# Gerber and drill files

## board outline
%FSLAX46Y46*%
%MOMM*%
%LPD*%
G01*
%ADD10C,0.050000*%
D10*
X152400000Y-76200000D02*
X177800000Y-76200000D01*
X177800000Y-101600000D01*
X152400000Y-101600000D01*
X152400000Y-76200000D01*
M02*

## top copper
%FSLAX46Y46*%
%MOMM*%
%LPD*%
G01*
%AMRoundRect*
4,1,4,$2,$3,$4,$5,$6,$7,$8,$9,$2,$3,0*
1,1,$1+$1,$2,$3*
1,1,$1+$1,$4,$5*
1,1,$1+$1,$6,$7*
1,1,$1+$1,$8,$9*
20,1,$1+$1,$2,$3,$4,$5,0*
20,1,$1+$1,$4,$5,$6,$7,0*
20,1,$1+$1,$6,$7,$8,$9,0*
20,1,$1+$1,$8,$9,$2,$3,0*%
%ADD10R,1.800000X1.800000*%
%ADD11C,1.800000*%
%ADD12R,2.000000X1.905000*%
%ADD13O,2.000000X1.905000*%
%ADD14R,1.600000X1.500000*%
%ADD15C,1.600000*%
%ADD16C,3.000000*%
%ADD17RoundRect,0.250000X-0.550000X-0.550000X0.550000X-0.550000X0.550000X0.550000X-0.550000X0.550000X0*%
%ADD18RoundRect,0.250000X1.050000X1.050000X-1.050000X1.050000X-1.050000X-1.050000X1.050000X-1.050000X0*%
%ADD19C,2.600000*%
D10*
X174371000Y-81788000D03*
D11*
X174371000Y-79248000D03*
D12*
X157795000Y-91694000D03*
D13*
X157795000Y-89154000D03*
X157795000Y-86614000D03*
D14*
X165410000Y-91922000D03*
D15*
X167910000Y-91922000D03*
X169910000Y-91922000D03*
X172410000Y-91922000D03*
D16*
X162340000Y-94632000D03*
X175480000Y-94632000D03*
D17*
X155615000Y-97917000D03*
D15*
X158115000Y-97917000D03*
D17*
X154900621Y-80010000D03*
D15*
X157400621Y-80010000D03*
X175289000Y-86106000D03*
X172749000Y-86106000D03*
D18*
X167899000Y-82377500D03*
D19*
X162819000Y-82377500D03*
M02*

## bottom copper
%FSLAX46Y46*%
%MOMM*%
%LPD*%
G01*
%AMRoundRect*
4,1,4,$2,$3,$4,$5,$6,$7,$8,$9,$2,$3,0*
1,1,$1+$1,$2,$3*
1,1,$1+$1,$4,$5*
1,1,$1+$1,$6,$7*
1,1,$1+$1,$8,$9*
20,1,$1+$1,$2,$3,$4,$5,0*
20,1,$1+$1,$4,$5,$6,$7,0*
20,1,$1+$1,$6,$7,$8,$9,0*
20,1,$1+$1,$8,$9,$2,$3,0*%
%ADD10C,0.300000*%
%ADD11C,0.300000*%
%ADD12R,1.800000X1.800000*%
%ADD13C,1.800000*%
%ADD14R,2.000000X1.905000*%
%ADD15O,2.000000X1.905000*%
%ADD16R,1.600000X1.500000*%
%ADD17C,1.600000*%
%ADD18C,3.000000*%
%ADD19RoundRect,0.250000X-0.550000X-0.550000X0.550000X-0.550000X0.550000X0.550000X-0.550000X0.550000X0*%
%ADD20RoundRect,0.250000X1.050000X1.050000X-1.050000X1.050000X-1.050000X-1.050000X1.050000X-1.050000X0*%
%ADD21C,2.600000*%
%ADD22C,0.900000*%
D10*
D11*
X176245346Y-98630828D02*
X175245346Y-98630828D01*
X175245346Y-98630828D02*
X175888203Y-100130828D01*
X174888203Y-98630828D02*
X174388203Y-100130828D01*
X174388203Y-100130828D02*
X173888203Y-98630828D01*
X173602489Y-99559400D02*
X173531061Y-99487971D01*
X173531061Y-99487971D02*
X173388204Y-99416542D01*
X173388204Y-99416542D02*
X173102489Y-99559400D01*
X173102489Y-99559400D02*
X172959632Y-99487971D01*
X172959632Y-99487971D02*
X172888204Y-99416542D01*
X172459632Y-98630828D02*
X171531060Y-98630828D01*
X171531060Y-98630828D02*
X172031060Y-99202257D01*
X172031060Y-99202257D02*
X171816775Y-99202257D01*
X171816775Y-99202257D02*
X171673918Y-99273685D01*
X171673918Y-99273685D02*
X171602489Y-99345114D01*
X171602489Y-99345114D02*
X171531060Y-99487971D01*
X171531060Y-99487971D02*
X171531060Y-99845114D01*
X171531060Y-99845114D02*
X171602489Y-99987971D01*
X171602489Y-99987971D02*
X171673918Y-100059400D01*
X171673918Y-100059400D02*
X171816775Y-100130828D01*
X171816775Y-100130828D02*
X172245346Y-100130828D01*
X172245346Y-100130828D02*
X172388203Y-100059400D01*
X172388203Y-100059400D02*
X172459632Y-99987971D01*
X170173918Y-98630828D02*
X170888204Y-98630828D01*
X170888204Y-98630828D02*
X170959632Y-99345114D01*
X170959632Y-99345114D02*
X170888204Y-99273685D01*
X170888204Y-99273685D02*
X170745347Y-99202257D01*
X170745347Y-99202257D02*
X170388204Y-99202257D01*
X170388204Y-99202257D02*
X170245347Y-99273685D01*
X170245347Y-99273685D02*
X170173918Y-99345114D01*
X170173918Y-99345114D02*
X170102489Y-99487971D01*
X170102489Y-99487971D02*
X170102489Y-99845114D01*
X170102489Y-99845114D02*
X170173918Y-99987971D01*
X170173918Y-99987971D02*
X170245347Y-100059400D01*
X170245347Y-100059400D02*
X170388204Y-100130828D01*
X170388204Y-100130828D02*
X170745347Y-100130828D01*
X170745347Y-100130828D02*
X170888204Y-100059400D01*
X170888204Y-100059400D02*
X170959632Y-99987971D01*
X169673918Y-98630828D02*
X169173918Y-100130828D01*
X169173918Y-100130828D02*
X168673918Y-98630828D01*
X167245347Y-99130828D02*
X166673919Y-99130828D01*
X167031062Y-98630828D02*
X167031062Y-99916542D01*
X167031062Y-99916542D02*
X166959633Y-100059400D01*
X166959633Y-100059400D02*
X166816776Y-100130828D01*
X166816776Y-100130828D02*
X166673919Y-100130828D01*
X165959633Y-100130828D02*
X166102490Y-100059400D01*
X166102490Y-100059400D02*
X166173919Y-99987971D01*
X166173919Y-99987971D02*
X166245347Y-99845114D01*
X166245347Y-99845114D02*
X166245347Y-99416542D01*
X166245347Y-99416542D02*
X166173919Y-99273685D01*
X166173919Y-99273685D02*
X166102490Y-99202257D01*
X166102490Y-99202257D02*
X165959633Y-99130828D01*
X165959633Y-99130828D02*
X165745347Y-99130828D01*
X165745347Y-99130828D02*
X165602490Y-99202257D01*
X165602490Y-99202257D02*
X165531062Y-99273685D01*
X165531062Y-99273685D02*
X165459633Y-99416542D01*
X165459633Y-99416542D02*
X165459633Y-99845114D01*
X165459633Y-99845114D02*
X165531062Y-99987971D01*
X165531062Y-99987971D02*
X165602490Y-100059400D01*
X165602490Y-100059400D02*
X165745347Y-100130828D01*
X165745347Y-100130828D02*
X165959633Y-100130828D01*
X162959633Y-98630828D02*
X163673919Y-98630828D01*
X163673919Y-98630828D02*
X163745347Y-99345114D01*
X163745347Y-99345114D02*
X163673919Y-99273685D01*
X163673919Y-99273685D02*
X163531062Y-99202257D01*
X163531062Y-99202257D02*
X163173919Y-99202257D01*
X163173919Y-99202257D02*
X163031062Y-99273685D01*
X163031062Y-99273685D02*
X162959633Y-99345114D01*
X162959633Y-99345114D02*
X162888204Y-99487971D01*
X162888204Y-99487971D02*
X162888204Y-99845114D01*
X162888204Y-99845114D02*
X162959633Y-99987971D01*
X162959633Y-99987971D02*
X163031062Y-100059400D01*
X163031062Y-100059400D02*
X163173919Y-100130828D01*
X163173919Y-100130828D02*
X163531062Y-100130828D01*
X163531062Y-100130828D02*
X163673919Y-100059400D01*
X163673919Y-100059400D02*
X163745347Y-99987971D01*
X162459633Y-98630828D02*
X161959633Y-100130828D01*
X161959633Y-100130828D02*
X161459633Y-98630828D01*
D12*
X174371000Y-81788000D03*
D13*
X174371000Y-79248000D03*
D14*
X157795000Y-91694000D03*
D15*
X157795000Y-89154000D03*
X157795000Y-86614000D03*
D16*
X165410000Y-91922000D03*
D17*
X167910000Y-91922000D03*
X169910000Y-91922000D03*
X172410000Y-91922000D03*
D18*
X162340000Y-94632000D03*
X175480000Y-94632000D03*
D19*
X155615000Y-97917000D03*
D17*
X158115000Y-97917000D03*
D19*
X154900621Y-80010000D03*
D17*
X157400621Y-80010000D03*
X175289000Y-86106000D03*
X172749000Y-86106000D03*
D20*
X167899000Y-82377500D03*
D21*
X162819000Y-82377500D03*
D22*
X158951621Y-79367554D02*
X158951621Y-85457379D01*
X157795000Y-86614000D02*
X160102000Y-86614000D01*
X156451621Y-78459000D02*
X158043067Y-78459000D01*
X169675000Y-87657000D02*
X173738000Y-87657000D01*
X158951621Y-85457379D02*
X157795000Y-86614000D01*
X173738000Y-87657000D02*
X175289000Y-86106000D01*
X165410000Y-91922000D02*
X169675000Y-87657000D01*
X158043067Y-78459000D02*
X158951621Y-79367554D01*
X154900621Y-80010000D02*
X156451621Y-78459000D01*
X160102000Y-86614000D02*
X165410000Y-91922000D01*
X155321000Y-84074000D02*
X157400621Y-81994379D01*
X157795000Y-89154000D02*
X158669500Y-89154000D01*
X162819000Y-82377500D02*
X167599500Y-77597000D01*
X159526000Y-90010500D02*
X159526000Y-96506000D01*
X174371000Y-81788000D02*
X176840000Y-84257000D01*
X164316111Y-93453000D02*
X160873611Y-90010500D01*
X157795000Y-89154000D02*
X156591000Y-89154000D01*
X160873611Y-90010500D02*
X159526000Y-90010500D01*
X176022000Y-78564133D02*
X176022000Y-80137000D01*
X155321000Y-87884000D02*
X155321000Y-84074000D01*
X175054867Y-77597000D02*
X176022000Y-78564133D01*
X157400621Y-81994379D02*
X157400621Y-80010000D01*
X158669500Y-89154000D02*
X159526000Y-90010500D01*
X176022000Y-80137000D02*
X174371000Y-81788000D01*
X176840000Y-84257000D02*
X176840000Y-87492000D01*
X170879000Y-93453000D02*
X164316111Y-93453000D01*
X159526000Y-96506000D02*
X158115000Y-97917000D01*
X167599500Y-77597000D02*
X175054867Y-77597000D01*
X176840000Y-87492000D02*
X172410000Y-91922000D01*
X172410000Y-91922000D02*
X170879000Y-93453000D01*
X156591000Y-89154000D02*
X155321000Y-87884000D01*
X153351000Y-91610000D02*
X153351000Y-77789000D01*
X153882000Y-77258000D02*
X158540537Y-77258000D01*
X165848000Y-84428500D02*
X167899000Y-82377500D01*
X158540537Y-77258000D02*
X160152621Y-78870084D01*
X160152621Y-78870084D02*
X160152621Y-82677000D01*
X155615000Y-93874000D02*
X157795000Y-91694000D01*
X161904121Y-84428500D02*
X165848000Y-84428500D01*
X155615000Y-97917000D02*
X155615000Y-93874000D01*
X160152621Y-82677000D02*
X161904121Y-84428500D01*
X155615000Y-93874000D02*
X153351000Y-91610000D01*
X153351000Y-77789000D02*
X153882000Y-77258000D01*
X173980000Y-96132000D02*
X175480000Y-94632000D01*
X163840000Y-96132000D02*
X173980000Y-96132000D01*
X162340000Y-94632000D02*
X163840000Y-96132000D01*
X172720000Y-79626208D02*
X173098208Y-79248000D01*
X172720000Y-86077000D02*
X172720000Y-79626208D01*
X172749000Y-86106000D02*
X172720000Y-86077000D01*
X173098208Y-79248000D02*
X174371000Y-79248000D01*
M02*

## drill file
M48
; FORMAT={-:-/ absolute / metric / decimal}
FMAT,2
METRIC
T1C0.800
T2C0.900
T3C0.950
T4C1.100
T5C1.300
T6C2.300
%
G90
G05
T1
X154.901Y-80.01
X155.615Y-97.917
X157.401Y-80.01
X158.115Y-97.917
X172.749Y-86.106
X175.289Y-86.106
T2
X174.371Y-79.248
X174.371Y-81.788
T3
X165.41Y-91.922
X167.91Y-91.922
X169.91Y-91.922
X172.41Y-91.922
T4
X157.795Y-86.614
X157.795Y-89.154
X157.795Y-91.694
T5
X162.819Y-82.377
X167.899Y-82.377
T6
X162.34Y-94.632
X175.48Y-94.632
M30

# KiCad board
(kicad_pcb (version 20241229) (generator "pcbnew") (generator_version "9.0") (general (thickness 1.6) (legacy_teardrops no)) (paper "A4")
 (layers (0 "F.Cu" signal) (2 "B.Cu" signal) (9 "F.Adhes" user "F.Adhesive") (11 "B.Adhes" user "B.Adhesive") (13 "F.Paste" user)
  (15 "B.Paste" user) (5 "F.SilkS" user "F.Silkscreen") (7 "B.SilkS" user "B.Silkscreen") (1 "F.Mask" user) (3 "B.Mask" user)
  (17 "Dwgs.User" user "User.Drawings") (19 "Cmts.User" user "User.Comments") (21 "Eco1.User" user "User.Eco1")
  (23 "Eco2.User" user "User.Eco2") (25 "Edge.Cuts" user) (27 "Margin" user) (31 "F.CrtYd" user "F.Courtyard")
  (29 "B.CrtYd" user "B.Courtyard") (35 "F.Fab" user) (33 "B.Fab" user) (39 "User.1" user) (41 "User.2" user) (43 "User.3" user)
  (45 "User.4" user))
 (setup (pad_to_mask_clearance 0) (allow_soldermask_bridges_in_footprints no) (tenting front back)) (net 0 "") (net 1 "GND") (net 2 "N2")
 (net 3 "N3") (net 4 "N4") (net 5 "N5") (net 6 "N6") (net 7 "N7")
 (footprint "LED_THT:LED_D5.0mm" (layer "F.Cu") (at 174.371 81.788 90)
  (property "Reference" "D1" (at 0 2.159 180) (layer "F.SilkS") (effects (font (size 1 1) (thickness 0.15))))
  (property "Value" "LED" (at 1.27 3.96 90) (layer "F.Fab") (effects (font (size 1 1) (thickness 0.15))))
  (pad "1" thru_hole rect (at 0 0 90) (size 1.8 1.8) (drill 0.9) (layers "*.Cu" "*.Mask") (remove_unused_layers no) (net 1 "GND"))
  (pad "2" thru_hole circle (at 2.54 0 90) (size 1.8 1.8) (drill 0.9) (layers "*.Cu" "*.Mask") (remove_unused_layers no) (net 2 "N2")))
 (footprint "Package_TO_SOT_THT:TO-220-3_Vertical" (layer "F.Cu") (at 157.795 91.694 90)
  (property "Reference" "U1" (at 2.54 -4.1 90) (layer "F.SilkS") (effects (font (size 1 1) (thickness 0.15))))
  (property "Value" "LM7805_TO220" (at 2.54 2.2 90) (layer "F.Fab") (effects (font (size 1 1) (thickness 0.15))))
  (pad "1" thru_hole rect (at 0 0 90) (size 1.905 2) (drill 1.1) (layers "*.Cu" "*.Mask") (remove_unused_layers no) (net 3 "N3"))
  (pad "2" thru_hole oval (at 2.54 0 90) (size 1.905 2) (drill 1.1) (layers "*.Cu" "*.Mask") (remove_unused_layers no) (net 1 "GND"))
  (pad "3" thru_hole oval (at 5.08 0 90) (size 1.905 2) (drill 1.1) (layers "*.Cu" "*.Mask") (remove_unused_layers no) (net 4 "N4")))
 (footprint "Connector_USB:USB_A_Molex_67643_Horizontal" (layer "F.Cu") (at 165.41 91.922)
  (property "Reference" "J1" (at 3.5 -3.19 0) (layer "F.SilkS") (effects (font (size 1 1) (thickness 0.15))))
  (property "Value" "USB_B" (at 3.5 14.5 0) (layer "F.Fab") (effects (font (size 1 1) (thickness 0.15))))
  (pad "1" thru_hole rect (at 0 0) (size 1.6 1.5) (drill 0.95) (layers "*.Cu" "*.Mask") (remove_unused_layers no) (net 4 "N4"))
  (pad "2" thru_hole circle (at 2.5 0) (size 1.6 1.6) (drill 0.95) (layers "*.Cu" "*.Mask") (remove_unused_layers no) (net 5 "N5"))
  (pad "3" thru_hole circle (at 4.5 0) (size 1.6 1.6) (drill 0.95) (layers "*.Cu" "*.Mask") (remove_unused_layers no) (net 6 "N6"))
  (pad "4" thru_hole circle (at 7 0) (size 1.6 1.6) (drill 0.95) (layers "*.Cu" "*.Mask") (remove_unused_layers no) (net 1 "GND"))
  (pad "5" thru_hole circle (at -3.07 2.71) (size 3 3) (drill 2.3) (layers "*.Cu" "*.Mask") (remove_unused_layers no) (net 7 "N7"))
  (pad "5" thru_hole circle (at 10.07 2.71) (size 3 3) (drill 2.3) (layers "*.Cu" "*.Mask") (remove_unused_layers no) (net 7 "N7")))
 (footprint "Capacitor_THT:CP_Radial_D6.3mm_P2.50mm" (layer "F.Cu") (at 155.615 97.917)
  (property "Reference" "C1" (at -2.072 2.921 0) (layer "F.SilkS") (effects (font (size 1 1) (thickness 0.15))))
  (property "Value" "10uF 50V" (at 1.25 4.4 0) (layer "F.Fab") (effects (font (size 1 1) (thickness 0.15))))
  (pad "1" thru_hole roundrect (at 0 0) (size 1.6 1.6) (drill 0.8) (layers "*.Cu" "*.Mask") (remove_unused_layers no)
   (roundrect_rratio 0.15625) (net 3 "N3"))
  (pad "2" thru_hole circle (at 2.5 0) (size 1.6 1.6) (drill 0.8) (layers "*.Cu" "*.Mask") (remove_unused_layers no) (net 1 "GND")))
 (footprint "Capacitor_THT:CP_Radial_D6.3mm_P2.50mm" (layer "F.Cu") (at 154.900621 80.01)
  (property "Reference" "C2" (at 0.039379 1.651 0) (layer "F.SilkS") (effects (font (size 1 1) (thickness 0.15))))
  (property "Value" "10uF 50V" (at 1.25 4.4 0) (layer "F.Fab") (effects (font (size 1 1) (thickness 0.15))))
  (pad "1" thru_hole roundrect (at 0 0) (size 1.6 1.6) (drill 0.8) (layers "*.Cu" "*.Mask") (remove_unused_layers no)
   (roundrect_rratio 0.15625) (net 4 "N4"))
  (pad "2" thru_hole circle (at 2.5 0) (size 1.6 1.6) (drill 0.8) (layers "*.Cu" "*.Mask") (remove_unused_layers no) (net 1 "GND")))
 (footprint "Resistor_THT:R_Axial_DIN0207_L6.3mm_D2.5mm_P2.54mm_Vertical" (layer "F.Cu") (at 175.289 86.106 180)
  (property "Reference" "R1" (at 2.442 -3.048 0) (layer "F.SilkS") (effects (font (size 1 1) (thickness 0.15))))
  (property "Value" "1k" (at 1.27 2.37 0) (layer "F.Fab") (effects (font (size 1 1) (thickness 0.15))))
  (pad "1" thru_hole circle (at 0 0 180) (size 1.6 1.6) (drill 0.8) (layers "*.Cu" "*.Mask") (remove_unused_layers no) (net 4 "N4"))
  (pad "2" thru_hole circle (at 2.54 0 180) (size 1.6 1.6) (drill 0.8) (layers "*.Cu" "*.Mask") (remove_unused_layers no) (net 2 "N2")))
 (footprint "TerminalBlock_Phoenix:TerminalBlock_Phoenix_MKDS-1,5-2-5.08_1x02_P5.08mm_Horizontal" (layer "F.Cu") (at 167.899 82.3775 180)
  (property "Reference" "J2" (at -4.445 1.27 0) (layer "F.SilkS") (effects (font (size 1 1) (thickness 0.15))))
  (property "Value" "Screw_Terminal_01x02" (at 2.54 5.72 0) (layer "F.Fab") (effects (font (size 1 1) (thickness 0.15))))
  (pad "1" thru_hole roundrect (at 0 0 180) (size 2.6 2.6) (drill 1.3) (layers "*.Cu" "*.Mask") (remove_unused_layers no)
   (roundrect_rratio 0.096154) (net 3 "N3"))
  (pad "2" thru_hole circle (at 5.08 0 180) (size 2.6 2.6) (drill 1.3) (layers "*.Cu" "*.Mask") (remove_unused_layers no) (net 1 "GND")))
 (gr_rect (start 152.4 76.2) (end 177.8 101.6) (stroke (width 0.05) (type default)) (fill no) (layer "Edge.Cuts"))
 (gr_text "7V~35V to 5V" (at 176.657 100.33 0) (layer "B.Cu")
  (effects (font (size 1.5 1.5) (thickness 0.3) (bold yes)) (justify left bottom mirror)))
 (segment (start 158.951621 79.367554) (end 158.951621 85.457379) (width 0.9) (layer "B.Cu") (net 4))
 (segment (start 157.795 86.614) (end 160.102 86.614) (width 0.9) (layer "B.Cu") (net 4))
 (segment (start 156.451621 78.459) (end 158.043067 78.459) (width 0.9) (layer "B.Cu") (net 4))
 (segment (start 169.675 87.657) (end 173.738 87.657) (width 0.9) (layer "B.Cu") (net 4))
 (segment (start 158.951621 85.457379) (end 157.795 86.614) (width 0.9) (layer "B.Cu") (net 4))
 (segment (start 173.738 87.657) (end 175.289 86.106) (width 0.9) (layer "B.Cu") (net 4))
 (segment (start 165.41 91.922) (end 169.675 87.657) (width 0.9) (layer "B.Cu") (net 4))
 (segment (start 158.043067 78.459) (end 158.951621 79.367554) (width 0.9) (layer "B.Cu") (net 4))
 (segment (start 154.900621 80.01) (end 156.451621 78.459) (width 0.9) (layer "B.Cu") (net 4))
 (segment (start 160.102 86.614) (end 165.41 91.922) (width 0.9) (layer "B.Cu") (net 4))
 (segment (start 155.321 84.074) (end 157.400621 81.994379) (width 0.9) (layer "B.Cu") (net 1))
 (segment (start 157.795 89.154) (end 158.6695 89.154) (width 0.9) (layer "B.Cu") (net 1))
 (segment (start 162.819 82.3775) (end 167.5995 77.597) (width 0.9) (layer "B.Cu") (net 1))
 (segment (start 159.526 90.0105) (end 159.526 96.506) (width 0.9) (layer "B.Cu") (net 1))
 (segment (start 174.371 81.788) (end 176.84 84.257) (width 0.9) (layer "B.Cu") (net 1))
 (segment (start 164.316111 93.453) (end 160.873611 90.0105) (width 0.9) (layer "B.Cu") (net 1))
 (segment (start 157.795 89.154) (end 156.591 89.154) (width 0.9) (layer "B.Cu") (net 1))
 (segment (start 160.873611 90.0105) (end 159.526 90.0105) (width 0.9) (layer "B.Cu") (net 1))
 (segment (start 176.022 78.564133) (end 176.022 80.137) (width 0.9) (layer "B.Cu") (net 1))
 (segment (start 155.321 87.884) (end 155.321 84.074) (width 0.9) (layer "B.Cu") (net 1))
 (segment (start 175.054867 77.597) (end 176.022 78.564133) (width 0.9) (layer "B.Cu") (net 1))
 (segment (start 157.400621 81.994379) (end 157.400621 80.01) (width 0.9) (layer "B.Cu") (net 1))
 (segment (start 158.6695 89.154) (end 159.526 90.0105) (width 0.9) (layer "B.Cu") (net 1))
 (segment (start 176.022 80.137) (end 174.371 81.788) (width 0.9) (layer "B.Cu") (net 1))
 (segment (start 176.84 84.257) (end 176.84 87.492) (width 0.9) (layer "B.Cu") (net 1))
 (segment (start 170.879 93.453) (end 164.316111 93.453) (width 0.9) (layer "B.Cu") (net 1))
 (segment (start 159.526 96.506) (end 158.115 97.917) (width 0.9) (layer "B.Cu") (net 1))
 (segment (start 167.5995 77.597) (end 175.054867 77.597) (width 0.9) (layer "B.Cu") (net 1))
 (segment (start 176.84 87.492) (end 172.41 91.922) (width 0.9) (layer "B.Cu") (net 1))
 (segment (start 172.41 91.922) (end 170.879 93.453) (width 0.9) (layer "B.Cu") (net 1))
 (segment (start 156.591 89.154) (end 155.321 87.884) (width 0.9) (layer "B.Cu") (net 1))
 (segment (start 153.351 91.61) (end 153.351 77.789) (width 0.9) (layer "B.Cu") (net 3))
 (segment (start 153.882 77.258) (end 158.540537 77.258) (width 0.9) (layer "B.Cu") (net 3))
 (segment (start 165.848 84.4285) (end 167.899 82.3775) (width 0.9) (layer "B.Cu") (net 3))
 (segment (start 158.540537 77.258) (end 160.152621 78.870084) (width 0.9) (layer "B.Cu") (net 3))
 (segment (start 160.152621 78.870084) (end 160.152621 82.677) (width 0.9) (layer "B.Cu") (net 3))
 (segment (start 155.615 93.874) (end 157.795 91.694) (width 0.9) (layer "B.Cu") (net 3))
 (segment (start 161.904121 84.4285) (end 165.848 84.4285) (width 0.9) (layer "B.Cu") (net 3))
 (segment (start 155.615 97.917) (end 155.615 93.874) (width 0.9) (layer "B.Cu") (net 3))
 (segment (start 160.152621 82.677) (end 161.904121 84.4285) (width 0.9) (layer "B.Cu") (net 3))
 (segment (start 155.615 93.874) (end 153.351 91.61) (width 0.9) (layer "B.Cu") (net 3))
 (segment (start 153.351 77.789) (end 153.882 77.258) (width 0.9) (layer "B.Cu") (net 3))
 (segment (start 173.98 96.132) (end 175.48 94.632) (width 0.9) (layer "B.Cu") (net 7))
 (segment (start 163.84 96.132) (end 173.98 96.132) (width 0.9) (layer "B.Cu") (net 7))
 (segment (start 162.34 94.632) (end 163.84 96.132) (width 0.9) (layer "B.Cu") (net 7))
 (segment (start 172.72 79.626208) (end 173.098208 79.248) (width 0.9) (layer "B.Cu") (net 2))
 (segment (start 172.72 86.077) (end 172.72 79.626208) (width 0.9) (layer "B.Cu") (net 2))
 (segment (start 172.749 86.106) (end 172.72 86.077) (width 0.9) (layer "B.Cu") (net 2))
 (segment (start 173.098208 79.248) (end 174.371 79.248) (width 0.9) (layer "B.Cu") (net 2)))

